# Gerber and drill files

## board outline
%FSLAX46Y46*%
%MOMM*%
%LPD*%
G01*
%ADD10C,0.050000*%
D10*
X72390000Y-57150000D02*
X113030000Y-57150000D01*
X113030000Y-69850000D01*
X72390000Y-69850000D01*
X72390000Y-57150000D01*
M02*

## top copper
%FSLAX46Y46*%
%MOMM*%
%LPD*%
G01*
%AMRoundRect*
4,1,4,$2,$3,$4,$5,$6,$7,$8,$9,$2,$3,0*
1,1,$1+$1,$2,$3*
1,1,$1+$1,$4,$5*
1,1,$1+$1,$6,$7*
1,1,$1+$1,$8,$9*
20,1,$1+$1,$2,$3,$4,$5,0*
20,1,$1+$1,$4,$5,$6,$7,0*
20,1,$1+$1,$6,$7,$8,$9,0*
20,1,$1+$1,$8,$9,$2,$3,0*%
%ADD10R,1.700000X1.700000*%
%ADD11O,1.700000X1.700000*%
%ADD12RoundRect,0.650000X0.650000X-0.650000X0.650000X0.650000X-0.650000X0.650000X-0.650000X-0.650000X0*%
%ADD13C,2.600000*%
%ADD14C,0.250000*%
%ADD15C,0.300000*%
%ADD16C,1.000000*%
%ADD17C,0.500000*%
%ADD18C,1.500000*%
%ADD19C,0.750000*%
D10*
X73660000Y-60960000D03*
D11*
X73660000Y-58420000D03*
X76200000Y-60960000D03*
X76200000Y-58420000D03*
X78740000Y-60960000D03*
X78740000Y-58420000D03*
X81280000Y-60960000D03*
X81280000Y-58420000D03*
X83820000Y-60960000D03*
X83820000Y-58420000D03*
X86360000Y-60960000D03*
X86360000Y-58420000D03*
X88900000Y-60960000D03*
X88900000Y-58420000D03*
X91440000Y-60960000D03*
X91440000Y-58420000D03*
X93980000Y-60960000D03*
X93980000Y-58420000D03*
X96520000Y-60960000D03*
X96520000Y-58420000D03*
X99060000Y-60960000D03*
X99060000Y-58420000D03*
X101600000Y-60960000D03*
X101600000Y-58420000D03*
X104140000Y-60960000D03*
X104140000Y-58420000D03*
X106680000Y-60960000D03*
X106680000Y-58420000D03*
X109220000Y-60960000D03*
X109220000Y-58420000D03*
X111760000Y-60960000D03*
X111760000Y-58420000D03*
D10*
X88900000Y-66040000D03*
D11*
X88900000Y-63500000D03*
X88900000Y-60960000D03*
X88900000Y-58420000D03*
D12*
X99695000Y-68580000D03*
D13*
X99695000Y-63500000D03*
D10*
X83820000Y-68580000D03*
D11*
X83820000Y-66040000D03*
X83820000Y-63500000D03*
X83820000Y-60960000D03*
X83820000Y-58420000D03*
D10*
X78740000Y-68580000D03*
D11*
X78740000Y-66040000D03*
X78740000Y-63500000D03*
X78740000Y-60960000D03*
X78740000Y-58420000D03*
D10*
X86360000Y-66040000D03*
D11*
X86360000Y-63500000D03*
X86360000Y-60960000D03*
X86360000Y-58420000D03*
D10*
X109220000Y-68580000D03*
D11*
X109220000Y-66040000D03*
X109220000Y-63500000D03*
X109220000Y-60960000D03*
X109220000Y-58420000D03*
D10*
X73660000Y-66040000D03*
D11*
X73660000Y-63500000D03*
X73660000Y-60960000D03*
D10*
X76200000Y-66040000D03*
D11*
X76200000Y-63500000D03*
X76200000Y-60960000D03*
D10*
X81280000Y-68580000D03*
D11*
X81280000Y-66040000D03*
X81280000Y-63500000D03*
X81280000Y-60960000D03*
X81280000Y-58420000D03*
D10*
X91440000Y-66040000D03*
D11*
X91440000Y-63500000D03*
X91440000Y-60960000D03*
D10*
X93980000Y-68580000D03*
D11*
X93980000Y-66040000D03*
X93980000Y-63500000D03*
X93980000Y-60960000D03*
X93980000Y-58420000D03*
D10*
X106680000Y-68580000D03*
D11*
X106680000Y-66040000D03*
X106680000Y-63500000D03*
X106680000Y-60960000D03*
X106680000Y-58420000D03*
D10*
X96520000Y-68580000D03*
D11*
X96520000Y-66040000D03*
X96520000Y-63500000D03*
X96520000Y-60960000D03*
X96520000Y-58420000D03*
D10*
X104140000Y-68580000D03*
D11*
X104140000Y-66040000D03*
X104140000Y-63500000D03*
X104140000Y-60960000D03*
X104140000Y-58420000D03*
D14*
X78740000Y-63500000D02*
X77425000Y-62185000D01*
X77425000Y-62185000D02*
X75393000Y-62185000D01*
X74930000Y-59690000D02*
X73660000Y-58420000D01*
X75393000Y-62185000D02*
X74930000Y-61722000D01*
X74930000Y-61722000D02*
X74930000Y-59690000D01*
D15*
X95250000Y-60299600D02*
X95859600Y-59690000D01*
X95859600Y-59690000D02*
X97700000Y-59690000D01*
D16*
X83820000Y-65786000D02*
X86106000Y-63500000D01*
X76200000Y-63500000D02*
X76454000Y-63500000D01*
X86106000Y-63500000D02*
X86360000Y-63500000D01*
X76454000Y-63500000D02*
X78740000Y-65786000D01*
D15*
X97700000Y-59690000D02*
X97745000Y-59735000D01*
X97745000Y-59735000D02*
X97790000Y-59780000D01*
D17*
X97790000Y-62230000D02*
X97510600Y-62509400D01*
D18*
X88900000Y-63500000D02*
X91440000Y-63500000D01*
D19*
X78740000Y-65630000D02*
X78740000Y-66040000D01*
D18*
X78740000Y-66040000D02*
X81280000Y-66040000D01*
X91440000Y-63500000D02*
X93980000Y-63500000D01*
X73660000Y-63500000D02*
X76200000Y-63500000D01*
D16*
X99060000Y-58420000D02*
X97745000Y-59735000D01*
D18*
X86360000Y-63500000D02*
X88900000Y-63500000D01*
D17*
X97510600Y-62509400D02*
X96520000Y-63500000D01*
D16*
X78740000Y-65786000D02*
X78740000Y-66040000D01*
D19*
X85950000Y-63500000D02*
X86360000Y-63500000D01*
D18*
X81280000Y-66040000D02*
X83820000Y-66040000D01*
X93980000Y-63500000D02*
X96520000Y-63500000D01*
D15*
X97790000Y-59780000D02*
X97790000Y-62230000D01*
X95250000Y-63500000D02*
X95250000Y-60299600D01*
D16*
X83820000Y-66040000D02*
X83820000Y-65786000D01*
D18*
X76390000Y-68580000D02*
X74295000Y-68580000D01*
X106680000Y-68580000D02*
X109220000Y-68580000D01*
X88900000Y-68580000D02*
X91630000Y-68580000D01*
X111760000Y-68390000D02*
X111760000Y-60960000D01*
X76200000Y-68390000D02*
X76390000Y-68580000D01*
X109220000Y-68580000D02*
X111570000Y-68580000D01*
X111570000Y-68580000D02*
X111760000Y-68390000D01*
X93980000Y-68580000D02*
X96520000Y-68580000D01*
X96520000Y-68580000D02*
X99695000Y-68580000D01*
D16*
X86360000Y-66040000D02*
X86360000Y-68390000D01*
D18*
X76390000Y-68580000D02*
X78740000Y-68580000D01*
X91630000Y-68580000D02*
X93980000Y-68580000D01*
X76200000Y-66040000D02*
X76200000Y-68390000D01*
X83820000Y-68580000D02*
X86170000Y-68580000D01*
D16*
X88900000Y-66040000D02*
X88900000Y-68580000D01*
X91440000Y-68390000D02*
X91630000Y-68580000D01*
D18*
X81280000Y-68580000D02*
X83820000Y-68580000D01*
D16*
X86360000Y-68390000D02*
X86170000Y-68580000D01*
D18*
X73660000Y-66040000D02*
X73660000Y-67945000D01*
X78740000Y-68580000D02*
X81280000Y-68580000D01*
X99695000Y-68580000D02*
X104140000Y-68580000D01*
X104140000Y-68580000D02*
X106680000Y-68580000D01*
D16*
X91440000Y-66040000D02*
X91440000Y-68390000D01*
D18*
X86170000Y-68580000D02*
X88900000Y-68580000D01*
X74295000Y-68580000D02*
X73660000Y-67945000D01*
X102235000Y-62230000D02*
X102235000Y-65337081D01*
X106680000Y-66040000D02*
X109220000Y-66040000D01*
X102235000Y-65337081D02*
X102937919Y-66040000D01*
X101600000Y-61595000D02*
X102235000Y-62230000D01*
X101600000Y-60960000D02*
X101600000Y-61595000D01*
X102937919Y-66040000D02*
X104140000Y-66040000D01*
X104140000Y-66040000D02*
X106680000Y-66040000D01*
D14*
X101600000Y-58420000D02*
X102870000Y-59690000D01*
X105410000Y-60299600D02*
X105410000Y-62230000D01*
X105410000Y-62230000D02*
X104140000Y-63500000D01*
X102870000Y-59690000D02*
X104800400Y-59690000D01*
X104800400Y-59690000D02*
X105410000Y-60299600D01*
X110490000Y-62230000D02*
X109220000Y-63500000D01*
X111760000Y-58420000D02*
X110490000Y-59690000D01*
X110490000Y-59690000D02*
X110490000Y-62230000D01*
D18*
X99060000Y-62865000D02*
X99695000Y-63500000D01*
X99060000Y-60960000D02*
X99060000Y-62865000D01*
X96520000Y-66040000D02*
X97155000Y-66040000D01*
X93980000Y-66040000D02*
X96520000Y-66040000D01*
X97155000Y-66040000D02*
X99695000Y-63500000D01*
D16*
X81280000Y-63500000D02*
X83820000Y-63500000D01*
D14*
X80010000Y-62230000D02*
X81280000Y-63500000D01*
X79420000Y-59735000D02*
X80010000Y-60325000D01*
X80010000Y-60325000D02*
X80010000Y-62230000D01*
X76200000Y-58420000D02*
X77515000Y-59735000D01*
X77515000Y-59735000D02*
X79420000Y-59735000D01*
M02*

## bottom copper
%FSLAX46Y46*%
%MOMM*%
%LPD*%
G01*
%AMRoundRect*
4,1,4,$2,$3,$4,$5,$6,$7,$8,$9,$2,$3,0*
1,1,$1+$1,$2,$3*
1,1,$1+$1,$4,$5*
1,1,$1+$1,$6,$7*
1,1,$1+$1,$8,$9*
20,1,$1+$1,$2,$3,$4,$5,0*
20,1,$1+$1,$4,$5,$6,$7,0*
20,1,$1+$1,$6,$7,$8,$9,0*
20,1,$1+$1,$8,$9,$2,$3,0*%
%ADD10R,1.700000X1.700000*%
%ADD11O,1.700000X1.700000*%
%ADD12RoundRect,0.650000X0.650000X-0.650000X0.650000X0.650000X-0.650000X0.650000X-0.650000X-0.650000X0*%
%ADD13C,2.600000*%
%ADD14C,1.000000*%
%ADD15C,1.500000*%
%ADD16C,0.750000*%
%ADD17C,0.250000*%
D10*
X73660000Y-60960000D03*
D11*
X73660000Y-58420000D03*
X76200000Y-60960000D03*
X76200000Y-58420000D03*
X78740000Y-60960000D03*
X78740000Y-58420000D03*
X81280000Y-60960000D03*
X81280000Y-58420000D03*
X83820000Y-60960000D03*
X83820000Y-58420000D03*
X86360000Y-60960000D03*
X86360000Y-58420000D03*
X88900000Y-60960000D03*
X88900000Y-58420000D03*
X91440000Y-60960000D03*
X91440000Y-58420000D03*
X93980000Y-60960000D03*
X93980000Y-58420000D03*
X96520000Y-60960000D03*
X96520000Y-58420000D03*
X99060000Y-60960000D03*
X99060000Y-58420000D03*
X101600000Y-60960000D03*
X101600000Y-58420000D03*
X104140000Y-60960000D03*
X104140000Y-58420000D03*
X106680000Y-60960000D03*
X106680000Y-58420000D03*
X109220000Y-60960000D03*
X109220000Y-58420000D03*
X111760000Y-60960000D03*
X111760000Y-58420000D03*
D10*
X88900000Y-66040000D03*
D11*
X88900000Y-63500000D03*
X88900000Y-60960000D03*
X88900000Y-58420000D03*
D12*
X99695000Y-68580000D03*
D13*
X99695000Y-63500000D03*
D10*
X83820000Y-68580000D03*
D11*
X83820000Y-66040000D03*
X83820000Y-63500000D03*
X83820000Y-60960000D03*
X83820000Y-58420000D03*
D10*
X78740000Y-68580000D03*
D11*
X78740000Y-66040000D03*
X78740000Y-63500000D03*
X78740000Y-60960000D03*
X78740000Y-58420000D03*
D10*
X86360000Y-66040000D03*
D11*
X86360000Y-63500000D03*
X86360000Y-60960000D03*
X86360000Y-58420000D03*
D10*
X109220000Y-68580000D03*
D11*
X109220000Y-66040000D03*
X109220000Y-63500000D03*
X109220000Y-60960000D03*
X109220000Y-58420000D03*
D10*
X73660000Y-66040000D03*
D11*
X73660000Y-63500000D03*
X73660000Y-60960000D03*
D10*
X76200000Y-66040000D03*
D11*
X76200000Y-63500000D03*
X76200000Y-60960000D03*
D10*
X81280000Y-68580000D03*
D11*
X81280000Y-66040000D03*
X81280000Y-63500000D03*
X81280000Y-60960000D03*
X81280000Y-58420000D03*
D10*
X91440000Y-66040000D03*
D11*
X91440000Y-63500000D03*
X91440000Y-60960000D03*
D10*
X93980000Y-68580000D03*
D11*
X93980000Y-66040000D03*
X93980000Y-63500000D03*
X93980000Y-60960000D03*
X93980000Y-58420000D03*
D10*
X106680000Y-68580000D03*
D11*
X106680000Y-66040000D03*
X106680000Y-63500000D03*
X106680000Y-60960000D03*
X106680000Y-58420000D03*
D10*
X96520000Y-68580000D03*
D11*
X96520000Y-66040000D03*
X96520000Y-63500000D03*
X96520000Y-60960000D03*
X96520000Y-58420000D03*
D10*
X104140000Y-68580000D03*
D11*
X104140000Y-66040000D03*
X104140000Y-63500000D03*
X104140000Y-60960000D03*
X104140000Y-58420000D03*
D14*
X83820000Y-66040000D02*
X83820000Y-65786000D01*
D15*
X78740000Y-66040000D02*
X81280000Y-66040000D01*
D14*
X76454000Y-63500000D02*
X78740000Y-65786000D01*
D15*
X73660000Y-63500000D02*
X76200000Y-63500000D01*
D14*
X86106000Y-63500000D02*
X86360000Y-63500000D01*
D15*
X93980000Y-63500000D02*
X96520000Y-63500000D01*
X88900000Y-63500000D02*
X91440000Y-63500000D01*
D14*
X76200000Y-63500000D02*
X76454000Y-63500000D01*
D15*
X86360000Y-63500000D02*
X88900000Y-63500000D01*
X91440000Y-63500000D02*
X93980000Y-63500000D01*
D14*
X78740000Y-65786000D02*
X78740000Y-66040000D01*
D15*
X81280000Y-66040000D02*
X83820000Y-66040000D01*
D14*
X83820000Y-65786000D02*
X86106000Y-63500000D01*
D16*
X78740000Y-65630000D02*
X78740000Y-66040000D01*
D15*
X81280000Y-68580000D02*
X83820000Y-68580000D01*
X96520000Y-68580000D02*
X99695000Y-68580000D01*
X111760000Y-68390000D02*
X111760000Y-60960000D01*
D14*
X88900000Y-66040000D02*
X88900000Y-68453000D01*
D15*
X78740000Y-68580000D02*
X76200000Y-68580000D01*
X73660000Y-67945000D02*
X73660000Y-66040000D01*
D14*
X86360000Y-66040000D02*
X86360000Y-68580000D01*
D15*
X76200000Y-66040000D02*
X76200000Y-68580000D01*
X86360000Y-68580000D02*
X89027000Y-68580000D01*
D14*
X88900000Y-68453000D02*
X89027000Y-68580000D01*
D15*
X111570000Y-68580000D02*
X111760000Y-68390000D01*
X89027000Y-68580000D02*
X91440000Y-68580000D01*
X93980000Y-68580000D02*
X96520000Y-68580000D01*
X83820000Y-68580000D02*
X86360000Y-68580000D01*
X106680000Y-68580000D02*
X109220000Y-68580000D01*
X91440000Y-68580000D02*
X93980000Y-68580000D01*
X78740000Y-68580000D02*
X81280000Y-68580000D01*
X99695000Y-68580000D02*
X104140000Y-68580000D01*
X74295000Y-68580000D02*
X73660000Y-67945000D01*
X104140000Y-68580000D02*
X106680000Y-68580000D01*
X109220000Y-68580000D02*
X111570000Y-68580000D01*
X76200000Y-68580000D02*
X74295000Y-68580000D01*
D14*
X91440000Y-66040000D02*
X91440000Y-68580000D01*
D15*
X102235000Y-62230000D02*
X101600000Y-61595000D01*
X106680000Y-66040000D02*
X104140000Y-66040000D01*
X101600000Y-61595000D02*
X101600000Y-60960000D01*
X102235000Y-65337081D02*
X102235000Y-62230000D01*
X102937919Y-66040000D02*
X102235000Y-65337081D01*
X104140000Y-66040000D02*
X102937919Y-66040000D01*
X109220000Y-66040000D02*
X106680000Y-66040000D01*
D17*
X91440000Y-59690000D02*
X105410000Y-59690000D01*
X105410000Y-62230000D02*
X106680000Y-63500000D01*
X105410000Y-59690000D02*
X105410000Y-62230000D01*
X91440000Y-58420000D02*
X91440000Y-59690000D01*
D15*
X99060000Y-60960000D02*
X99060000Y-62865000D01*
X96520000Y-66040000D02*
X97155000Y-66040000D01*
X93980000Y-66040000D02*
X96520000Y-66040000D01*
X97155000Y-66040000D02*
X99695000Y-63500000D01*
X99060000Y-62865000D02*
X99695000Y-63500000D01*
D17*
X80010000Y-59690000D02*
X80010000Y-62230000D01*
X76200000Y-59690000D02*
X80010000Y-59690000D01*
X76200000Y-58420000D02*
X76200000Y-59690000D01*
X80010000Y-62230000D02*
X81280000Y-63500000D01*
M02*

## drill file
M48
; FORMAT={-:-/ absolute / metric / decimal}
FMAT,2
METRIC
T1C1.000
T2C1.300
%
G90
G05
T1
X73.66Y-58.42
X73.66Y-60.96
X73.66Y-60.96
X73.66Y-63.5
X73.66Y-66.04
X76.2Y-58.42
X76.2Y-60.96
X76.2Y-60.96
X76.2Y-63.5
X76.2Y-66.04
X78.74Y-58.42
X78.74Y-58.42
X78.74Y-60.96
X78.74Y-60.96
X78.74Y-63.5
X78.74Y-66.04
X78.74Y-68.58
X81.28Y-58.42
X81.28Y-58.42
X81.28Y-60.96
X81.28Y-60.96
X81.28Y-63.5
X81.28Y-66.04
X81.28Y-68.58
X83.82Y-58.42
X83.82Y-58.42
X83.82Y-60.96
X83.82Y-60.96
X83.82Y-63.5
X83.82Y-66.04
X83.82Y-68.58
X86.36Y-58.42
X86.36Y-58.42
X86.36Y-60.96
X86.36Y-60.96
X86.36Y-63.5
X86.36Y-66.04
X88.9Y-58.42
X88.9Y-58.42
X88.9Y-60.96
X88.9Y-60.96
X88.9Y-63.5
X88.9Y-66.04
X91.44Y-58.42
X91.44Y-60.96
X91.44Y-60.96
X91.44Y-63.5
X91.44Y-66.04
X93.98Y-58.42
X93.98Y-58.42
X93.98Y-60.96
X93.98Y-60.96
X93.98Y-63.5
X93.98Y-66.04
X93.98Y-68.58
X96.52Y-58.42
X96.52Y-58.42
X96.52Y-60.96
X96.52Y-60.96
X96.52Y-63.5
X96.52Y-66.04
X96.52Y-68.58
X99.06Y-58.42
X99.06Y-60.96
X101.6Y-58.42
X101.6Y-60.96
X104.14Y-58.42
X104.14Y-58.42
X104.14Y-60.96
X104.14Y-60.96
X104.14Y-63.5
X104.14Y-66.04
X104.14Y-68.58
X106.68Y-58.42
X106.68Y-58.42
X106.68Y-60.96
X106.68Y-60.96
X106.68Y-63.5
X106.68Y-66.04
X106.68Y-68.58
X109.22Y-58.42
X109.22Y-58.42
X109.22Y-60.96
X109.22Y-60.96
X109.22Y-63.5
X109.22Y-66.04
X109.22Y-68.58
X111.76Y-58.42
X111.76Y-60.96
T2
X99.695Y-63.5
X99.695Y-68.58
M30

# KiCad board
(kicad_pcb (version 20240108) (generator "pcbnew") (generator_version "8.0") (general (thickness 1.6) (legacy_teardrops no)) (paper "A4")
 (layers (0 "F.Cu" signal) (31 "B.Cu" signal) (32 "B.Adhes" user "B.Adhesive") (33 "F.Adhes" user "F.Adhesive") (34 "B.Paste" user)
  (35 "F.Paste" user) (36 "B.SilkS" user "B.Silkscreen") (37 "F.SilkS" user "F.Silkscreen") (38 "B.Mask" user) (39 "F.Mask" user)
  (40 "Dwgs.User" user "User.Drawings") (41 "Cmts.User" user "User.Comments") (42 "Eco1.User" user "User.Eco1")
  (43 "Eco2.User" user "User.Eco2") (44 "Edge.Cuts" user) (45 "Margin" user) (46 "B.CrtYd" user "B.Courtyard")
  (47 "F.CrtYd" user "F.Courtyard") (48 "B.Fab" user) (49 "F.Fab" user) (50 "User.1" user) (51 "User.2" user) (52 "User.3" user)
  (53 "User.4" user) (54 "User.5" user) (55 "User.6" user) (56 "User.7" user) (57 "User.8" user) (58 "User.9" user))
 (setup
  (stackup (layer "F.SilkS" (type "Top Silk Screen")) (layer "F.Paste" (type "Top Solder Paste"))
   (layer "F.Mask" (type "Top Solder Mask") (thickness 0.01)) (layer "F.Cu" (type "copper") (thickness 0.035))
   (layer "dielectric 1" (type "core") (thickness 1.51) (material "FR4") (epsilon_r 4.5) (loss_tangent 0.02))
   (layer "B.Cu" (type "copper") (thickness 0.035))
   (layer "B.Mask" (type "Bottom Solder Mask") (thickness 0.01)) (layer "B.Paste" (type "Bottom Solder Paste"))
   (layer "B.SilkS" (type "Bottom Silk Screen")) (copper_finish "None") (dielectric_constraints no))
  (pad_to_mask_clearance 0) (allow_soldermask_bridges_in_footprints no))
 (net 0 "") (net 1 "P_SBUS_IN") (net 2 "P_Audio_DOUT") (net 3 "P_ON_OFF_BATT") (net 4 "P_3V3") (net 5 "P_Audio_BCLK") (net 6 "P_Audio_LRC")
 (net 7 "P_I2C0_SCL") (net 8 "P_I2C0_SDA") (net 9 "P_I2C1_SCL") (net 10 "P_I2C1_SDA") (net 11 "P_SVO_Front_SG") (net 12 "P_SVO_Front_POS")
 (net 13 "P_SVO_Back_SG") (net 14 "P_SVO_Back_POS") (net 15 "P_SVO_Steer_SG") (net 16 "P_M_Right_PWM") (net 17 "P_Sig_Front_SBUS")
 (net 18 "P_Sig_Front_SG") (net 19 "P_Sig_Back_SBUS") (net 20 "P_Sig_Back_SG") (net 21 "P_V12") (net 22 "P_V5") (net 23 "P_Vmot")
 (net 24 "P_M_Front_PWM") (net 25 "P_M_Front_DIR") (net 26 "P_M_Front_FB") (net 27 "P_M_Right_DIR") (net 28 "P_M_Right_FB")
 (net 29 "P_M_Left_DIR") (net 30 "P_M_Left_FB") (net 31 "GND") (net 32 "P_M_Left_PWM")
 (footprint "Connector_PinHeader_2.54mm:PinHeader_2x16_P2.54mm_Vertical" (layer "F.Cu") (at 73.66 60.96 90)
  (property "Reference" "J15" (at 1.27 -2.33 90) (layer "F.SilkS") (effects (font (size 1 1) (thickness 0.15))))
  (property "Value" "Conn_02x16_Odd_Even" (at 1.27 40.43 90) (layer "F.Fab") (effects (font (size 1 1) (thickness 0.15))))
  (pad "1" thru_hole rect (at 0 0 90) (size 1.7 1.7) (drill 1) (layers "*.Cu" "*.Mask") (remove_unused_layers no) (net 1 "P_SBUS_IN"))
  (pad "2" thru_hole oval (at 2.54 0 90) (size 1.7 1.7) (drill 1) (layers "*.Cu" "*.Mask") (remove_unused_layers no) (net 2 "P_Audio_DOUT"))
  (pad "3" thru_hole oval (at 0 2.54 90) (size 1.7 1.7) (drill 1) (layers "*.Cu" "*.Mask") (remove_unused_layers no) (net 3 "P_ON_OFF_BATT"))
  (pad "4" thru_hole oval (at 2.54 2.54 90) (size 1.7 1.7) (drill 1) (layers "*.Cu" "*.Mask") (remove_unused_layers no) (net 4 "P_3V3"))
  (pad "5" thru_hole oval (at 0 5.08 90) (size 1.7 1.7) (drill 1) (layers "*.Cu" "*.Mask") (remove_unused_layers no) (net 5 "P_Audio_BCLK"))
  (pad "6" thru_hole oval (at 2.54 5.08 90) (size 1.7 1.7) (drill 1) (layers "*.Cu" "*.Mask") (remove_unused_layers no)
   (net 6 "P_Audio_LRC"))
  (pad "7" thru_hole oval (at 0 7.62 90) (size 1.7 1.7) (drill 1) (layers "*.Cu" "*.Mask") (remove_unused_layers no) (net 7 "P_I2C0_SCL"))
  (pad "8" thru_hole oval (at 2.54 7.62 90) (size 1.7 1.7) (drill 1) (layers "*.Cu" "*.Mask") (remove_unused_layers no) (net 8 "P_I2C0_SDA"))
  (pad "9" thru_hole oval (at 0 10.16 90) (size 1.7 1.7) (drill 1) (layers "*.Cu" "*.Mask") (remove_unused_layers no) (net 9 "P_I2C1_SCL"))
  (pad "10" thru_hole oval (at 2.54 10.16 90) (size 1.7 1.7) (drill 1) (layers "*.Cu" "*.Mask") (remove_unused_layers no)
   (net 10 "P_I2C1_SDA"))
  (pad "11" thru_hole oval (at 0 12.7 90) (size 1.7 1.7) (drill 1) (layers "*.Cu" "*.Mask") (remove_unused_layers no)
   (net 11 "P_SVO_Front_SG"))
  (pad "12" thru_hole oval (at 2.54 12.7 90) (size 1.7 1.7) (drill 1) (layers "*.Cu" "*.Mask") (remove_unused_layers no)
   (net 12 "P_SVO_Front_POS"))
  (pad "13" thru_hole oval (at 0 15.24 90) (size 1.7 1.7) (drill 1) (layers "*.Cu" "*.Mask") (remove_unused_layers no)
   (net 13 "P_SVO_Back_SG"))
  (pad "14" thru_hole oval (at 2.54 15.24 90) (size 1.7 1.7) (drill 1) (layers "*.Cu" "*.Mask") (remove_unused_layers no)
   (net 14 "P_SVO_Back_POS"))
  (pad "15" thru_hole oval (at 0 17.78 90) (size 1.7 1.7) (drill 1) (layers "*.Cu" "*.Mask") (remove_unused_layers no)
   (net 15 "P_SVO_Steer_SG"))
  (pad "16" thru_hole oval (at 2.54 17.78 90) (size 1.7 1.7) (drill 1) (layers "*.Cu" "*.Mask") (remove_unused_layers no)
   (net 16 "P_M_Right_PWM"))
  (pad "17" thru_hole oval (at 0 20.32 90) (size 1.7 1.7) (drill 1) (layers "*.Cu" "*.Mask") (remove_unused_layers no)
   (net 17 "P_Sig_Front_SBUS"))
  (pad "18" thru_hole oval (at 2.54 20.32 90) (size 1.7 1.7) (drill 1) (layers "*.Cu" "*.Mask") (remove_unused_layers no)
   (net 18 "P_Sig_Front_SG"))
  (pad "19" thru_hole oval (at 0 22.86 90) (size 1.7 1.7) (drill 1) (layers "*.Cu" "*.Mask") (remove_unused_layers no)
   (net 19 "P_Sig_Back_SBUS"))
  (pad "20" thru_hole oval (at 2.54 22.86 90) (size 1.7 1.7) (drill 1) (layers "*.Cu" "*.Mask") (remove_unused_layers no)
   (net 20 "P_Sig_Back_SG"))
  (pad "21" thru_hole oval (at 0 25.4 90) (size 1.7 1.7) (drill 1) (layers "*.Cu" "*.Mask") (remove_unused_layers no) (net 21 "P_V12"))
  (pad "22" thru_hole oval (at 2.54 25.4 90) (size 1.7 1.7) (drill 1) (layers "*.Cu" "*.Mask") (remove_unused_layers no) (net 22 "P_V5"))
  (pad "23" thru_hole oval (at 0 27.94 90) (size 1.7 1.7) (drill 1) (layers "*.Cu" "*.Mask") (remove_unused_layers no) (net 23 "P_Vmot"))
  (pad "24" thru_hole oval (at 2.54 27.94 90) (size 1.7 1.7) (drill 1) (layers "*.Cu" "*.Mask") (remove_unused_layers no)
   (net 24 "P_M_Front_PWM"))
  (pad "25" thru_hole oval (at 0 30.48 90) (size 1.7 1.7) (drill 1) (layers "*.Cu" "*.Mask") (remove_unused_layers no)
   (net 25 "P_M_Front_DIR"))
  (pad "26" thru_hole oval (at 2.54 30.48 90) (size 1.7 1.7) (drill 1) (layers "*.Cu" "*.Mask") (remove_unused_layers no)
   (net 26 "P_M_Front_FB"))
  (pad "27" thru_hole oval (at 0 33.02 90) (size 1.7 1.7) (drill 1) (layers "*.Cu" "*.Mask") (remove_unused_layers no)
   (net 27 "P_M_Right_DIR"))
  (pad "28" thru_hole oval (at 2.54 33.02 90) (size 1.7 1.7) (drill 1) (layers "*.Cu" "*.Mask") (remove_unused_layers no)
   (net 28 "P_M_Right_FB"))
  (pad "29" thru_hole oval (at 0 35.56 90) (size 1.7 1.7) (drill 1) (layers "*.Cu" "*.Mask") (remove_unused_layers no)
   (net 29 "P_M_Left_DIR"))
  (pad "30" thru_hole oval (at 2.54 35.56 90) (size 1.7 1.7) (drill 1) (layers "*.Cu" "*.Mask") (remove_unused_layers no)
   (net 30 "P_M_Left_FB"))
  (pad "31" thru_hole oval (at 0 38.1 90) (size 1.7 1.7) (drill 1) (layers "*.Cu" "*.Mask") (remove_unused_layers no) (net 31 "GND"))
  (pad "32" thru_hole oval (at 2.54 38.1 90) (size 1.7 1.7) (drill 1) (layers "*.Cu" "*.Mask") (remove_unused_layers no)
   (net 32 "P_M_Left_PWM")))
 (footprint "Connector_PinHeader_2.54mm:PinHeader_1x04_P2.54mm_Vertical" (layer "F.Cu") (at 88.9 66.04 180)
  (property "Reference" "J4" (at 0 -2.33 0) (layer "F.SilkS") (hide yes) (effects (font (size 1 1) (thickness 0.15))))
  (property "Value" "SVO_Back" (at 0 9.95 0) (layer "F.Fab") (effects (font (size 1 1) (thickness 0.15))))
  (pad "1" thru_hole rect (at 0 0 180) (size 1.7 1.7) (drill 1) (layers "*.Cu" "*.Mask") (remove_unused_layers no) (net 31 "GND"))
  (pad "2" thru_hole oval (at 0 2.54 180) (size 1.7 1.7) (drill 1) (layers "*.Cu" "*.Mask") (remove_unused_layers no) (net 22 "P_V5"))
  (pad "3" thru_hole oval (at 0 5.08 180) (size 1.7 1.7) (drill 1) (layers "*.Cu" "*.Mask") (remove_unused_layers no)
   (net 13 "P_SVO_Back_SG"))
  (pad "4" thru_hole oval (at 0 7.62 180) (size 1.7 1.7) (drill 1) (layers "*.Cu" "*.Mask") (remove_unused_layers no)
   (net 14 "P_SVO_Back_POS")))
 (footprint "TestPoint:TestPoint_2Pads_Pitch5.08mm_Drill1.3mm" (layer "F.Cu") (at 99.695 68.58 90)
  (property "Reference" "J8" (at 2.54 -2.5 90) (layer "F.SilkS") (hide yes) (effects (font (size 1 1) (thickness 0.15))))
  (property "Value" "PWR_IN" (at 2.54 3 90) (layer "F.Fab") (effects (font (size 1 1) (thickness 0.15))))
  (pad "1" thru_hole roundrect (at 0 0 90) (size 2.6 2.6) (drill 1.3) (layers "*.Cu" "*.Mask") (remove_unused_layers no)
   (roundrect_rratio 0.25) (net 31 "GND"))
  (pad "2" thru_hole circle (at 5.08 0 90) (size 2.6 2.6) (drill 1.3) (layers "*.Cu" "*.Mask") (remove_unused_layers no) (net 21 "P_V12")))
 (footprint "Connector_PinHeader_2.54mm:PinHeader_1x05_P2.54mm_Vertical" (layer "F.Cu") (at 83.82 68.58 180)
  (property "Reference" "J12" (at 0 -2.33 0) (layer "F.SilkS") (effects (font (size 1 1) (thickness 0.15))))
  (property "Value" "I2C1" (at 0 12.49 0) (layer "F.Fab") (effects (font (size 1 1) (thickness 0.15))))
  (pad "1" thru_hole rect (at 0 0 180) (size 1.7 1.7) (drill 1) (layers "*.Cu" "*.Mask") (remove_unused_layers no) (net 31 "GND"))
  (pad "2" thru_hole oval (at 0 2.54 180) (size 1.7 1.7) (drill 1) (layers "*.Cu" "*.Mask") (remove_unused_layers no) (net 22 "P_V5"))
  (pad "3" thru_hole oval (at 0 5.08 180) (size 1.7 1.7) (drill 1) (layers "*.Cu" "*.Mask") (remove_unused_layers no) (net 4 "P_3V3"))
  (pad "4" thru_hole oval (at 0 7.62 180) (size 1.7 1.7) (drill 1) (layers "*.Cu" "*.Mask") (remove_unused_layers no) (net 9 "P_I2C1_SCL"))
  (pad "5" thru_hole oval (at 0 10.16 180) (size 1.7 1.7) (drill 1) (layers "*.Cu" "*.Mask") (remove_unused_layers no) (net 10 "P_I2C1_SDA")))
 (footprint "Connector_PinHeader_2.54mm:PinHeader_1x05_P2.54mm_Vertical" (layer "F.Cu") (at 78.74 68.58 180)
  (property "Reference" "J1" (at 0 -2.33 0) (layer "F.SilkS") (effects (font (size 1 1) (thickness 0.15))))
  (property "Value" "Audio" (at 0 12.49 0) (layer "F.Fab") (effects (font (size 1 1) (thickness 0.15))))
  (pad "1" thru_hole rect (at 0 0 180) (size 1.7 1.7) (drill 1) (layers "*.Cu" "*.Mask") (remove_unused_layers no) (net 31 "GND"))
  (pad "2" thru_hole oval (at 0 2.54 180) (size 1.7 1.7) (drill 1) (layers "*.Cu" "*.Mask") (remove_unused_layers no) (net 22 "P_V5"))
  (pad "3" thru_hole oval (at 0 5.08 180) (size 1.7 1.7) (drill 1) (layers "*.Cu" "*.Mask") (remove_unused_layers no) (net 2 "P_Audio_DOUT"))
  (pad "4" thru_hole oval (at 0 7.62 180) (size 1.7 1.7) (drill 1) (layers "*.Cu" "*.Mask") (remove_unused_layers no) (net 5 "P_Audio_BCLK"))
  (pad "5" thru_hole oval (at 0 10.16 180) (size 1.7 1.7) (drill 1) (layers "*.Cu" "*.Mask") (remove_unused_layers no) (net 6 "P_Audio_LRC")))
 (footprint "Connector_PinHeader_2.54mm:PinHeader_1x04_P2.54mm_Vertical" (layer "F.Cu") (at 86.36 66.04 180)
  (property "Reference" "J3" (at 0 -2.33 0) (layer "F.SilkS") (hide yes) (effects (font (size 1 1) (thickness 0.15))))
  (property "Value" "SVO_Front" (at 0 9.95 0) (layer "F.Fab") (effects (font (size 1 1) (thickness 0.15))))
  (pad "1" thru_hole rect (at 0 0 180) (size 1.7 1.7) (drill 1) (layers "*.Cu" "*.Mask") (remove_unused_layers no) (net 31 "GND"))
  (pad "2" thru_hole oval (at 0 2.54 180) (size 1.7 1.7) (drill 1) (layers "*.Cu" "*.Mask") (remove_unused_layers no) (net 22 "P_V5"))
  (pad "3" thru_hole oval (at 0 5.08 180) (size 1.7 1.7) (drill 1) (layers "*.Cu" "*.Mask") (remove_unused_layers no)
   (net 11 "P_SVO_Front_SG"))
  (pad "4" thru_hole oval (at 0 7.62 180) (size 1.7 1.7) (drill 1) (layers "*.Cu" "*.Mask") (remove_unused_layers no)
   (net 12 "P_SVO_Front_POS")))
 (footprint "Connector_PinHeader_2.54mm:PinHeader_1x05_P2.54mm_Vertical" (layer "F.Cu") (at 109.22 68.58 180)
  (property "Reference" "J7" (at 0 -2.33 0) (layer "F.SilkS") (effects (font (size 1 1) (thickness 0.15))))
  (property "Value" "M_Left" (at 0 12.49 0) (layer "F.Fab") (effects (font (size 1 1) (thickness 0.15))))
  (pad "1" thru_hole rect (at 0 0 180) (size 1.7 1.7) (drill 1) (layers "*.Cu" "*.Mask") (remove_unused_layers no) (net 31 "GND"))
  (pad "2" thru_hole oval (at 0 2.54 180) (size 1.7 1.7) (drill 1) (layers "*.Cu" "*.Mask") (remove_unused_layers no) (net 23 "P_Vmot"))
  (pad "3" thru_hole oval (at 0 5.08 180) (size 1.7 1.7) (drill 1) (layers "*.Cu" "*.Mask") (remove_unused_layers no)
   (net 32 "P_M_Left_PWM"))
  (pad "4" thru_hole oval (at 0 7.62 180) (size 1.7 1.7) (drill 1) (layers "*.Cu" "*.Mask") (remove_unused_layers no)
   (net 29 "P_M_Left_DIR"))
  (pad "5" thru_hole oval (at 0 10.16 180) (size 1.7 1.7) (drill 1) (layers "*.Cu" "*.Mask") (remove_unused_layers no)
   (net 30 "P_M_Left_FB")))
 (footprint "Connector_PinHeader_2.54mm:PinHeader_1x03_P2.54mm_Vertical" (layer "F.Cu") (at 73.66 66.04 180)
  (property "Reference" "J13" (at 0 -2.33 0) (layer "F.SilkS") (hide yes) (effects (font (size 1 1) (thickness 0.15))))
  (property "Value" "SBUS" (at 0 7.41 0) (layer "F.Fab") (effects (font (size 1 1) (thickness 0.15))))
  (pad "1" thru_hole rect (at 0 0 180) (size 1.7 1.7) (drill 1) (layers "*.Cu" "*.Mask") (remove_unused_layers no) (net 31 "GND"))
  (pad "2" thru_hole oval (at 0 2.54 180) (size 1.7 1.7) (drill 1) (layers "*.Cu" "*.Mask") (remove_unused_layers no) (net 22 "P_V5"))
  (pad "3" thru_hole oval (at 0 5.08 180) (size 1.7 1.7) (drill 1) (layers "*.Cu" "*.Mask") (remove_unused_layers no) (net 1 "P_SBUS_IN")))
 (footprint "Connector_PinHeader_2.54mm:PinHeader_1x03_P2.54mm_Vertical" (layer "F.Cu") (at 76.2 66.04 180)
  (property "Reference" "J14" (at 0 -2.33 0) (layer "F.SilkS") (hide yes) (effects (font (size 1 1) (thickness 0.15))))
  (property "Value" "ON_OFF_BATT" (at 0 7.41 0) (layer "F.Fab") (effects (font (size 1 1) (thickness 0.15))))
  (pad "1" thru_hole rect (at 0 0 180) (size 1.7 1.7) (drill 1) (layers "*.Cu" "*.Mask") (remove_unused_layers no) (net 31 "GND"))
  (pad "2" thru_hole oval (at 0 2.54 180) (size 1.7 1.7) (drill 1) (layers "*.Cu" "*.Mask") (remove_unused_layers no) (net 22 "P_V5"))
  (pad "3" thru_hole oval (at 0 5.08 180) (size 1.7 1.7) (drill 1) (layers "*.Cu" "*.Mask") (remove_unused_layers no)
   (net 3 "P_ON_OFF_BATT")))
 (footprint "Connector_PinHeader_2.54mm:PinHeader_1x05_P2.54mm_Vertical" (layer "F.Cu") (at 81.28 68.58 180)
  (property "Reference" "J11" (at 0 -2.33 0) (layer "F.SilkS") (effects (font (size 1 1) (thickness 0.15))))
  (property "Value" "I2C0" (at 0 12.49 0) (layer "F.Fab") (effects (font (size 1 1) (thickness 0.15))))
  (pad "1" thru_hole rect (at 0 0 180) (size 1.7 1.7) (drill 1) (layers "*.Cu" "*.Mask") (remove_unused_layers no) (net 31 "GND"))
  (pad "2" thru_hole oval (at 0 2.54 180) (size 1.7 1.7) (drill 1) (layers "*.Cu" "*.Mask") (remove_unused_layers no) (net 22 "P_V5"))
  (pad "3" thru_hole oval (at 0 5.08 180) (size 1.7 1.7) (drill 1) (layers "*.Cu" "*.Mask") (remove_unused_layers no) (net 4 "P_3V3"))
  (pad "4" thru_hole oval (at 0 7.62 180) (size 1.7 1.7) (drill 1) (layers "*.Cu" "*.Mask") (remove_unused_layers no) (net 7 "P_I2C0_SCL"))
  (pad "5" thru_hole oval (at 0 10.16 180) (size 1.7 1.7) (drill 1) (layers "*.Cu" "*.Mask") (remove_unused_layers no) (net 8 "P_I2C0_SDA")))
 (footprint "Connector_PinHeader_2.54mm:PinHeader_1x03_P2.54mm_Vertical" (layer "F.Cu") (at 91.44 66.04 180)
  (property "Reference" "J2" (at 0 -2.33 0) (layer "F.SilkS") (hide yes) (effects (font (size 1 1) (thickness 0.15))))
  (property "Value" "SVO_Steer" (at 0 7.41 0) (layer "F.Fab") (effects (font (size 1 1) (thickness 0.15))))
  (pad "1" thru_hole rect (at 0 0 180) (size 1.7 1.7) (drill 1) (layers "*.Cu" "*.Mask") (remove_unused_layers no) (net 31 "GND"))
  (pad "2" thru_hole oval (at 0 2.54 180) (size 1.7 1.7) (drill 1) (layers "*.Cu" "*.Mask") (remove_unused_layers no) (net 22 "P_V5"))
  (pad "3" thru_hole oval (at 0 5.08 180) (size 1.7 1.7) (drill 1) (layers "*.Cu" "*.Mask") (remove_unused_layers no)
   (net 15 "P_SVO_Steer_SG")))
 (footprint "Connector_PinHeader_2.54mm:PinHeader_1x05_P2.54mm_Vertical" (layer "F.Cu") (at 93.98 68.58 180)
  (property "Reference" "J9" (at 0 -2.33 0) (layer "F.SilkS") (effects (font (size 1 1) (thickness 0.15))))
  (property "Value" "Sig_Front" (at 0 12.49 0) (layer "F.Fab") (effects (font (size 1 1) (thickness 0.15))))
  (pad "1" thru_hole rect (at 0 0 180) (size 1.7 1.7) (drill 1) (layers "*.Cu" "*.Mask") (remove_unused_layers no) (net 31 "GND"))
  (pad "2" thru_hole oval (at 0 2.54 180) (size 1.7 1.7) (drill 1) (layers "*.Cu" "*.Mask") (remove_unused_layers no) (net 21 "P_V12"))
  (pad "3" thru_hole oval (at 0 5.08 180) (size 1.7 1.7) (drill 1) (layers "*.Cu" "*.Mask") (remove_unused_layers no) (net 22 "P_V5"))
  (pad "4" thru_hole oval (at 0 7.62 180) (size 1.7 1.7) (drill 1) (layers "*.Cu" "*.Mask") (remove_unused_layers no)
   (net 17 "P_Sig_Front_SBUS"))
  (pad "5" thru_hole oval (at 0 10.16 180) (size 1.7 1.7) (drill 1) (layers "*.Cu" "*.Mask") (remove_unused_layers no)
   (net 18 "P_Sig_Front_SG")))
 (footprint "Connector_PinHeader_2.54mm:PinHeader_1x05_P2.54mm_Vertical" (layer "F.Cu") (at 106.68 68.58 180)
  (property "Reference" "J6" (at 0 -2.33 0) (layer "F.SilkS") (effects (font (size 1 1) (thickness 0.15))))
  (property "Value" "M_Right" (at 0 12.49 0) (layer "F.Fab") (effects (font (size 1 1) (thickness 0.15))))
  (pad "1" thru_hole rect (at 0 0 180) (size 1.7 1.7) (drill 1) (layers "*.Cu" "*.Mask") (remove_unused_layers no) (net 31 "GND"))
  (pad "2" thru_hole oval (at 0 2.54 180) (size 1.7 1.7) (drill 1) (layers "*.Cu" "*.Mask") (remove_unused_layers no) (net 23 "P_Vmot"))
  (pad "3" thru_hole oval (at 0 5.08 180) (size 1.7 1.7) (drill 1) (layers "*.Cu" "*.Mask") (remove_unused_layers no)
   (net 16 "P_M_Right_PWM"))
  (pad "4" thru_hole oval (at 0 7.62 180) (size 1.7 1.7) (drill 1) (layers "*.Cu" "*.Mask") (remove_unused_layers no)
   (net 27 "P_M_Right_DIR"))
  (pad "5" thru_hole oval (at 0 10.16 180) (size 1.7 1.7) (drill 1) (layers "*.Cu" "*.Mask") (remove_unused_layers no)
   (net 28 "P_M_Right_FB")))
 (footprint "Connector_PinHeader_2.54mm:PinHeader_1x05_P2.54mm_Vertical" (layer "F.Cu") (at 96.52 68.58 180)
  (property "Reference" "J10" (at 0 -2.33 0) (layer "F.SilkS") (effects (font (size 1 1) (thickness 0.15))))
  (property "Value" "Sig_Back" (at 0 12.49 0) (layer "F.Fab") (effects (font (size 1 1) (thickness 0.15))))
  (pad "1" thru_hole rect (at 0 0 180) (size 1.7 1.7) (drill 1) (layers "*.Cu" "*.Mask") (remove_unused_layers no) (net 31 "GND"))
  (pad "2" thru_hole oval (at 0 2.54 180) (size 1.7 1.7) (drill 1) (layers "*.Cu" "*.Mask") (remove_unused_layers no) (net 21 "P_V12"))
  (pad "3" thru_hole oval (at 0 5.08 180) (size 1.7 1.7) (drill 1) (layers "*.Cu" "*.Mask") (remove_unused_layers no) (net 22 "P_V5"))
  (pad "4" thru_hole oval (at 0 7.62 180) (size 1.7 1.7) (drill 1) (layers "*.Cu" "*.Mask") (remove_unused_layers no)
   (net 19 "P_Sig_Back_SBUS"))
  (pad "5" thru_hole oval (at 0 10.16 180) (size 1.7 1.7) (drill 1) (layers "*.Cu" "*.Mask") (remove_unused_layers no)
   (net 20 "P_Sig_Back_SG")))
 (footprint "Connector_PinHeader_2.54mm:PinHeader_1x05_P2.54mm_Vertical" (layer "F.Cu") (at 104.14 68.58 180)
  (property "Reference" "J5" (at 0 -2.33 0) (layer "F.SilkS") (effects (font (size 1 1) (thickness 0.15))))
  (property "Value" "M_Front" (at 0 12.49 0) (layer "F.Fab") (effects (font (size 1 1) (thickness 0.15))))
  (pad "1" thru_hole rect (at 0 0 180) (size 1.7 1.7) (drill 1) (layers "*.Cu" "*.Mask") (remove_unused_layers no) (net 31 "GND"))
  (pad "2" thru_hole oval (at 0 2.54 180) (size 1.7 1.7) (drill 1) (layers "*.Cu" "*.Mask") (remove_unused_layers no) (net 23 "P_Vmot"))
  (pad "3" thru_hole oval (at 0 5.08 180) (size 1.7 1.7) (drill 1) (layers "*.Cu" "*.Mask") (remove_unused_layers no)
   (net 24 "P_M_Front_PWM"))
  (pad "4" thru_hole oval (at 0 7.62 180) (size 1.7 1.7) (drill 1) (layers "*.Cu" "*.Mask") (remove_unused_layers no)
   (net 25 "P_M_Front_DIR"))
  (pad "5" thru_hole oval (at 0 10.16 180) (size 1.7 1.7) (drill 1) (layers "*.Cu" "*.Mask") (remove_unused_layers no)
   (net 26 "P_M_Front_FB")))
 (gr_rect (start 72.39 57.15) (end 113.03 69.85) (stroke (width 0.05) (type default)) (fill none) (layer "Edge.Cuts"))
 (segment (start 78.74 63.5) (end 77.425 62.185) (width 0.25) (layer "F.Cu") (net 2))
 (segment (start 77.425 62.185) (end 75.393 62.185) (width 0.25) (layer "F.Cu") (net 2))
 (segment (start 74.93 59.69) (end 73.66 58.42) (width 0.25) (layer "F.Cu") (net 2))
 (segment (start 75.393 62.185) (end 74.93 61.722) (width 0.25) (layer "F.Cu") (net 2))
 (segment (start 74.93 61.722) (end 74.93 59.69) (width 0.25) (layer "F.Cu") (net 2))
 (segment (start 95.25 60.2996) (end 95.8596 59.69) (width 0.3) (layer "F.Cu") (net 22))
 (segment (start 95.8596 59.69) (end 97.7 59.69) (width 0.3) (layer "F.Cu") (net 22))
 (segment (start 83.82 65.786) (end 86.106 63.5) (width 1) (layer "F.Cu") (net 22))
 (segment (start 76.2 63.5) (end 76.454 63.5) (width 1) (layer "F.Cu") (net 22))
 (segment (start 86.106 63.5) (end 86.36 63.5) (width 1) (layer "F.Cu") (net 22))
 (segment (start 76.454 63.5) (end 78.74 65.786) (width 1) (layer "F.Cu") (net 22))
 (segment (start 97.7 59.69) (end 97.745 59.735) (width 0.3) (layer "F.Cu") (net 22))
 (segment (start 97.745 59.735) (end 97.79 59.78) (width 0.3) (layer "F.Cu") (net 22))
 (segment (start 97.79 62.23) (end 97.5106 62.5094) (width 0.5) (layer "F.Cu") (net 22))
 (segment (start 88.9 63.5) (end 91.44 63.5) (width 1.5) (layer "F.Cu") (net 22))
 (segment (start 78.74 65.63) (end 78.74 66.04) (width 0.75) (layer "F.Cu") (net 22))
 (segment (start 78.74 66.04) (end 81.28 66.04) (width 1.5) (layer "F.Cu") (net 22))
 (segment (start 91.44 63.5) (end 93.98 63.5) (width 1.5) (layer "F.Cu") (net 22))
 (segment (start 73.66 63.5) (end 76.2 63.5) (width 1.5) (layer "F.Cu") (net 22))
 (segment (start 99.06 58.42) (end 97.745 59.735) (width 1) (layer "F.Cu") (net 22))
 (segment (start 86.36 63.5) (end 88.9 63.5) (width 1.5) (layer "F.Cu") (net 22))
 (segment (start 97.5106 62.5094) (end 96.52 63.5) (width 0.5) (layer "F.Cu") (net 22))
 (segment (start 78.74 65.786) (end 78.74 66.04) (width 1) (layer "F.Cu") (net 22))
 (segment (start 85.95 63.5) (end 86.36 63.5) (width 0.75) (layer "F.Cu") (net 22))
 (segment (start 81.28 66.04) (end 83.82 66.04) (width 1.5) (layer "F.Cu") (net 22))
 (segment (start 93.98 63.5) (end 96.52 63.5) (width 1.5) (layer "F.Cu") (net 22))
 (segment (start 97.79 59.78) (end 97.79 62.23) (width 0.3) (layer "F.Cu") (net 22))
 (segment (start 95.25 63.5) (end 95.25 60.2996) (width 0.3) (layer "F.Cu") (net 22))
 (segment (start 83.82 66.04) (end 83.82 65.786) (width 1) (layer "F.Cu") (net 22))
 (segment (start 83.82 66.04) (end 83.82 65.786) (width 1) (layer "B.Cu") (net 22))
 (segment (start 78.74 66.04) (end 81.28 66.04) (width 1.5) (layer "B.Cu") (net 22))
 (segment (start 76.454 63.5) (end 78.74 65.786) (width 1) (layer "B.Cu") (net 22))
 (segment (start 73.66 63.5) (end 76.2 63.5) (width 1.5) (layer "B.Cu") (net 22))
 (segment (start 86.106 63.5) (end 86.36 63.5) (width 1) (layer "B.Cu") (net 22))
 (segment (start 93.98 63.5) (end 96.52 63.5) (width 1.5) (layer "B.Cu") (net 22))
 (segment (start 88.9 63.5) (end 91.44 63.5) (width 1.5) (layer "B.Cu") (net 22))
 (segment (start 76.2 63.5) (end 76.454 63.5) (width 1) (layer "B.Cu") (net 22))
 (segment (start 86.36 63.5) (end 88.9 63.5) (width 1.5) (layer "B.Cu") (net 22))
 (segment (start 91.44 63.5) (end 93.98 63.5) (width 1.5) (layer "B.Cu") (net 22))
 (segment (start 78.74 65.786) (end 78.74 66.04) (width 1) (layer "B.Cu") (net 22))
 (segment (start 81.28 66.04) (end 83.82 66.04) (width 1.5) (layer "B.Cu") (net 22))
 (segment (start 83.82 65.786) (end 86.106 63.5) (width 1) (layer "B.Cu") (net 22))
 (segment (start 78.74 65.63) (end 78.74 66.04) (width 0.75) (layer "B.Cu") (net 22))
 (segment (start 76.39 68.58) (end 74.295 68.58) (width 1.5) (layer "F.Cu") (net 31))
 (segment (start 106.68 68.58) (end 109.22 68.58) (width 1.5) (layer "F.Cu") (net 31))
 (segment (start 88.9 68.58) (end 91.63 68.58) (width 1.5) (layer "F.Cu") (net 31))
 (segment (start 111.76 68.39) (end 111.76 60.96) (width 1.5) (layer "F.Cu") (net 31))
 (segment (start 76.2 68.39) (end 76.39 68.58) (width 1.5) (layer "F.Cu") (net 31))
 (segment (start 109.22 68.58) (end 111.57 68.58) (width 1.5) (layer "F.Cu") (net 31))
 (segment (start 111.57 68.58) (end 111.76 68.39) (width 1.5) (layer "F.Cu") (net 31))
 (segment (start 93.98 68.58) (end 96.52 68.58) (width 1.5) (layer "F.Cu") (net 31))
 (segment (start 96.52 68.58) (end 99.695 68.58) (width 1.5) (layer "F.Cu") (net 31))
 (segment (start 86.36 66.04) (end 86.36 68.39) (width 1) (layer "F.Cu") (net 31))
 (segment (start 76.39 68.58) (end 78.74 68.58) (width 1.5) (layer "F.Cu") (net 31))
 (segment (start 91.63 68.58) (end 93.98 68.58) (width 1.5) (layer "F.Cu") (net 31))
 (segment (start 76.2 66.04) (end 76.2 68.39) (width 1.5) (layer "F.Cu") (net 31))
 (segment (start 83.82 68.58) (end 86.17 68.58) (width 1.5) (layer "F.Cu") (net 31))
 (segment (start 88.9 66.04) (end 88.9 68.58) (width 1) (layer "F.Cu") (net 31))
 (segment (start 91.44 68.39) (end 91.63 68.58) (width 1) (layer "F.Cu") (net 31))
 (segment (start 81.28 68.58) (end 83.82 68.58) (width 1.5) (layer "F.Cu") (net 31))
 (segment (start 86.36 68.39) (end 86.17 68.58) (width 1) (layer "F.Cu") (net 31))
 (segment (start 73.66 66.04) (end 73.66 67.945) (width 1.5) (layer "F.Cu") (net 31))
 (segment (start 78.74 68.58) (end 81.28 68.58) (width 1.5) (layer "F.Cu") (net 31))
 (segment (start 99.695 68.58) (end 104.14 68.58) (width 1.5) (layer "F.Cu") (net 31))
 (segment (start 104.14 68.58) (end 106.68 68.58) (width 1.5) (layer "F.Cu") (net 31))
 (segment (start 91.44 66.04) (end 91.44 68.39) (width 1) (layer "F.Cu") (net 31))
 (segment (start 86.17 68.58) (end 88.9 68.58) (width 1.5) (layer "F.Cu") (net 31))
 (segment (start 74.295 68.58) (end 73.66 67.945) (width 1.5) (layer "F.Cu") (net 31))
 (segment (start 81.28 68.58) (end 83.82 68.58) (width 1.5) (layer "B.Cu") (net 31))
 (segment (start 96.52 68.58) (end 99.695 68.58) (width 1.5) (layer "B.Cu") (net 31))
 (segment (start 111.76 68.39) (end 111.76 60.96) (width 1.5) (layer "B.Cu") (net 31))
 (segment (start 88.9 66.04) (end 88.9 68.453) (width 1) (layer "B.Cu") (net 31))
 (segment (start 78.74 68.58) (end 76.2 68.58) (width 1.5) (layer "B.Cu") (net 31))
 (segment (start 73.66 67.945) (end 73.66 66.04) (width 1.5) (layer "B.Cu") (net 31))
 (segment (start 86.36 66.04) (end 86.36 68.58) (width 1) (layer "B.Cu") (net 31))
 (segment (start 76.2 66.04) (end 76.2 68.58) (width 1.5) (layer "B.Cu") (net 31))
 (segment (start 86.36 68.58) (end 89.027 68.58) (width 1.5) (layer "B.Cu") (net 31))
 (segment (start 88.9 68.453) (end 89.027 68.58) (width 1) (layer "B.Cu") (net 31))
 (segment (start 111.57 68.58) (end 111.76 68.39) (width 1.5) (layer "B.Cu") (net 31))
 (segment (start 89.027 68.58) (end 91.44 68.58) (width 1.5) (layer "B.Cu") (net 31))
 (segment (start 93.98 68.58) (end 96.52 68.58) (width 1.5) (layer "B.Cu") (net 31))
 (segment (start 83.82 68.58) (end 86.36 68.58) (width 1.5) (layer "B.Cu") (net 31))
 (segment (start 106.68 68.58) (end 109.22 68.58) (width 1.5) (layer "B.Cu") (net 31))
 (segment (start 91.44 68.58) (end 93.98 68.58) (width 1.5) (layer "B.Cu") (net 31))
 (segment (start 78.74 68.58) (end 81.28 68.58) (width 1.5) (layer "B.Cu") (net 31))
 (segment (start 99.695 68.58) (end 104.14 68.58) (width 1.5) (layer "B.Cu") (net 31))
 (segment (start 74.295 68.58) (end 73.66 67.945) (width 1.5) (layer "B.Cu") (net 31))
 (segment (start 104.14 68.58) (end 106.68 68.58) (width 1.5) (layer "B.Cu") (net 31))
 (segment (start 109.22 68.58) (end 111.57 68.58) (width 1.5) (layer "B.Cu") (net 31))
 (segment (start 76.2 68.58) (end 74.295 68.58) (width 1.5) (layer "B.Cu") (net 31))
 (segment (start 91.44 66.04) (end 91.44 68.58) (width 1) (layer "B.Cu") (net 31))
 (segment (start 102.235 62.23) (end 102.235 65.337081) (width 1.5) (layer "F.Cu") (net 23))
 (segment (start 106.68 66.04) (end 109.22 66.04) (width 1.5) (layer "F.Cu") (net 23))
 (segment (start 102.235 65.337081) (end 102.937919 66.04) (width 1.5) (layer "F.Cu") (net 23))
 (segment (start 101.6 61.595) (end 102.235 62.23) (width 1.5) (layer "F.Cu") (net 23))
 (segment (start 101.6 60.96) (end 101.6 61.595) (width 1.5) (layer "F.Cu") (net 23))
 (segment (start 102.937919 66.04) (end 104.14 66.04) (width 1.5) (layer "F.Cu") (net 23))
 (segment (start 104.14 66.04) (end 106.68 66.04) (width 1.5) (layer "F.Cu") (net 23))
 (segment (start 102.235 62.23) (end 101.6 61.595) (width 1.5) (layer "B.Cu") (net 23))
 (segment (start 106.68 66.04) (end 104.14 66.04) (width 1.5) (layer "B.Cu") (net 23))
 (segment (start 101.6 61.595) (end 101.6 60.96) (width 1.5) (layer "B.Cu") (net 23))
 (segment (start 102.235 65.337081) (end 102.235 62.23) (width 1.5) (layer "B.Cu") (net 23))
 (segment (start 102.937919 66.04) (end 102.235 65.337081) (width 1.5) (layer "B.Cu") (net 23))
 (segment (start 104.14 66.04) (end 102.937919 66.04) (width 1.5) (layer "B.Cu") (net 23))
 (segment (start 109.22 66.04) (end 106.68 66.04) (width 1.5) (layer "B.Cu") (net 23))
 (segment (start 101.6 58.42) (end 102.87 59.69) (width 0.25) (layer "F.Cu") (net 24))
 (segment (start 105.41 60.2996) (end 105.41 62.23) (width 0.25) (layer "F.Cu") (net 24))
 (segment (start 105.41 62.23) (end 104.14 63.5) (width 0.25) (layer "F.Cu") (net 24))
 (segment (start 102.87 59.69) (end 104.8004 59.69) (width 0.25) (layer "F.Cu") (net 24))
 (segment (start 104.8004 59.69) (end 105.41 60.2996) (width 0.25) (layer "F.Cu") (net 24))
 (segment (start 91.44 59.69) (end 105.41 59.69) (width 0.25) (layer "B.Cu") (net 16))
 (segment (start 105.41 62.23) (end 106.68 63.5) (width 0.25) (layer "B.Cu") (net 16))
 (segment (start 105.41 59.69) (end 105.41 62.23) (width 0.25) (layer "B.Cu") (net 16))
 (segment (start 91.44 58.42) (end 91.44 59.69) (width 0.25) (layer "B.Cu") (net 16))
 (segment (start 110.49 62.23) (end 109.22 63.5) (width 0.25) (layer "F.Cu") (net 32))
 (segment (start 111.76 58.42) (end 110.49 59.69) (width 0.25) (layer "F.Cu") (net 32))
 (segment (start 110.49 59.69) (end 110.49 62.23) (width 0.25) (layer "F.Cu") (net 32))
 (segment (start 99.06 62.865) (end 99.695 63.5) (width 1.5) (layer "F.Cu") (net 21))
 (segment (start 99.06 60.96) (end 99.06 62.865) (width 1.5) (layer "F.Cu") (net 21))
 (segment (start 96.52 66.04) (end 97.155 66.04) (width 1.5) (layer "F.Cu") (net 21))
 (segment (start 93.98 66.04) (end 96.52 66.04) (width 1.5) (layer "F.Cu") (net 21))
 (segment (start 97.155 66.04) (end 99.695 63.5) (width 1.5) (layer "F.Cu") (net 21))
 (segment (start 99.06 60.96) (end 99.06 62.865) (width 1.5) (layer "B.Cu") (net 21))
 (segment (start 96.52 66.04) (end 97.155 66.04) (width 1.5) (layer "B.Cu") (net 21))
 (segment (start 93.98 66.04) (end 96.52 66.04) (width 1.5) (layer "B.Cu") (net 21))
 (segment (start 97.155 66.04) (end 99.695 63.5) (width 1.5) (layer "B.Cu") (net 21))
 (segment (start 99.06 62.865) (end 99.695 63.5) (width 1.5) (layer "B.Cu") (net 21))
 (segment (start 81.28 63.5) (end 83.82 63.5) (width 1) (layer "F.Cu") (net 4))
 (segment (start 80.01 62.23) (end 81.28 63.5) (width 0.25) (layer "F.Cu") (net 4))
 (segment (start 79.42 59.735) (end 80.01 60.325) (width 0.25) (layer "F.Cu") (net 4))
 (segment (start 80.01 60.325) (end 80.01 62.23) (width 0.25) (layer "F.Cu") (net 4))
 (segment (start 76.2 58.42) (end 77.515 59.735) (width 0.25) (layer "F.Cu") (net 4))
 (segment (start 77.515 59.735) (end 79.42 59.735) (width 0.25) (layer "F.Cu") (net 4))
 (segment (start 80.01 59.69) (end 80.01 62.23) (width 0.25) (layer "B.Cu") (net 4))
 (segment (start 76.2 59.69) (end 80.01 59.69) (width 0.25) (layer "B.Cu") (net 4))
 (segment (start 76.2 58.42) (end 76.2 59.69) (width 0.25) (layer "B.Cu") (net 4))
 (segment (start 80.01 62.23) (end 81.28 63.5) (width 0.25) (layer "B.Cu") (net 4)))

